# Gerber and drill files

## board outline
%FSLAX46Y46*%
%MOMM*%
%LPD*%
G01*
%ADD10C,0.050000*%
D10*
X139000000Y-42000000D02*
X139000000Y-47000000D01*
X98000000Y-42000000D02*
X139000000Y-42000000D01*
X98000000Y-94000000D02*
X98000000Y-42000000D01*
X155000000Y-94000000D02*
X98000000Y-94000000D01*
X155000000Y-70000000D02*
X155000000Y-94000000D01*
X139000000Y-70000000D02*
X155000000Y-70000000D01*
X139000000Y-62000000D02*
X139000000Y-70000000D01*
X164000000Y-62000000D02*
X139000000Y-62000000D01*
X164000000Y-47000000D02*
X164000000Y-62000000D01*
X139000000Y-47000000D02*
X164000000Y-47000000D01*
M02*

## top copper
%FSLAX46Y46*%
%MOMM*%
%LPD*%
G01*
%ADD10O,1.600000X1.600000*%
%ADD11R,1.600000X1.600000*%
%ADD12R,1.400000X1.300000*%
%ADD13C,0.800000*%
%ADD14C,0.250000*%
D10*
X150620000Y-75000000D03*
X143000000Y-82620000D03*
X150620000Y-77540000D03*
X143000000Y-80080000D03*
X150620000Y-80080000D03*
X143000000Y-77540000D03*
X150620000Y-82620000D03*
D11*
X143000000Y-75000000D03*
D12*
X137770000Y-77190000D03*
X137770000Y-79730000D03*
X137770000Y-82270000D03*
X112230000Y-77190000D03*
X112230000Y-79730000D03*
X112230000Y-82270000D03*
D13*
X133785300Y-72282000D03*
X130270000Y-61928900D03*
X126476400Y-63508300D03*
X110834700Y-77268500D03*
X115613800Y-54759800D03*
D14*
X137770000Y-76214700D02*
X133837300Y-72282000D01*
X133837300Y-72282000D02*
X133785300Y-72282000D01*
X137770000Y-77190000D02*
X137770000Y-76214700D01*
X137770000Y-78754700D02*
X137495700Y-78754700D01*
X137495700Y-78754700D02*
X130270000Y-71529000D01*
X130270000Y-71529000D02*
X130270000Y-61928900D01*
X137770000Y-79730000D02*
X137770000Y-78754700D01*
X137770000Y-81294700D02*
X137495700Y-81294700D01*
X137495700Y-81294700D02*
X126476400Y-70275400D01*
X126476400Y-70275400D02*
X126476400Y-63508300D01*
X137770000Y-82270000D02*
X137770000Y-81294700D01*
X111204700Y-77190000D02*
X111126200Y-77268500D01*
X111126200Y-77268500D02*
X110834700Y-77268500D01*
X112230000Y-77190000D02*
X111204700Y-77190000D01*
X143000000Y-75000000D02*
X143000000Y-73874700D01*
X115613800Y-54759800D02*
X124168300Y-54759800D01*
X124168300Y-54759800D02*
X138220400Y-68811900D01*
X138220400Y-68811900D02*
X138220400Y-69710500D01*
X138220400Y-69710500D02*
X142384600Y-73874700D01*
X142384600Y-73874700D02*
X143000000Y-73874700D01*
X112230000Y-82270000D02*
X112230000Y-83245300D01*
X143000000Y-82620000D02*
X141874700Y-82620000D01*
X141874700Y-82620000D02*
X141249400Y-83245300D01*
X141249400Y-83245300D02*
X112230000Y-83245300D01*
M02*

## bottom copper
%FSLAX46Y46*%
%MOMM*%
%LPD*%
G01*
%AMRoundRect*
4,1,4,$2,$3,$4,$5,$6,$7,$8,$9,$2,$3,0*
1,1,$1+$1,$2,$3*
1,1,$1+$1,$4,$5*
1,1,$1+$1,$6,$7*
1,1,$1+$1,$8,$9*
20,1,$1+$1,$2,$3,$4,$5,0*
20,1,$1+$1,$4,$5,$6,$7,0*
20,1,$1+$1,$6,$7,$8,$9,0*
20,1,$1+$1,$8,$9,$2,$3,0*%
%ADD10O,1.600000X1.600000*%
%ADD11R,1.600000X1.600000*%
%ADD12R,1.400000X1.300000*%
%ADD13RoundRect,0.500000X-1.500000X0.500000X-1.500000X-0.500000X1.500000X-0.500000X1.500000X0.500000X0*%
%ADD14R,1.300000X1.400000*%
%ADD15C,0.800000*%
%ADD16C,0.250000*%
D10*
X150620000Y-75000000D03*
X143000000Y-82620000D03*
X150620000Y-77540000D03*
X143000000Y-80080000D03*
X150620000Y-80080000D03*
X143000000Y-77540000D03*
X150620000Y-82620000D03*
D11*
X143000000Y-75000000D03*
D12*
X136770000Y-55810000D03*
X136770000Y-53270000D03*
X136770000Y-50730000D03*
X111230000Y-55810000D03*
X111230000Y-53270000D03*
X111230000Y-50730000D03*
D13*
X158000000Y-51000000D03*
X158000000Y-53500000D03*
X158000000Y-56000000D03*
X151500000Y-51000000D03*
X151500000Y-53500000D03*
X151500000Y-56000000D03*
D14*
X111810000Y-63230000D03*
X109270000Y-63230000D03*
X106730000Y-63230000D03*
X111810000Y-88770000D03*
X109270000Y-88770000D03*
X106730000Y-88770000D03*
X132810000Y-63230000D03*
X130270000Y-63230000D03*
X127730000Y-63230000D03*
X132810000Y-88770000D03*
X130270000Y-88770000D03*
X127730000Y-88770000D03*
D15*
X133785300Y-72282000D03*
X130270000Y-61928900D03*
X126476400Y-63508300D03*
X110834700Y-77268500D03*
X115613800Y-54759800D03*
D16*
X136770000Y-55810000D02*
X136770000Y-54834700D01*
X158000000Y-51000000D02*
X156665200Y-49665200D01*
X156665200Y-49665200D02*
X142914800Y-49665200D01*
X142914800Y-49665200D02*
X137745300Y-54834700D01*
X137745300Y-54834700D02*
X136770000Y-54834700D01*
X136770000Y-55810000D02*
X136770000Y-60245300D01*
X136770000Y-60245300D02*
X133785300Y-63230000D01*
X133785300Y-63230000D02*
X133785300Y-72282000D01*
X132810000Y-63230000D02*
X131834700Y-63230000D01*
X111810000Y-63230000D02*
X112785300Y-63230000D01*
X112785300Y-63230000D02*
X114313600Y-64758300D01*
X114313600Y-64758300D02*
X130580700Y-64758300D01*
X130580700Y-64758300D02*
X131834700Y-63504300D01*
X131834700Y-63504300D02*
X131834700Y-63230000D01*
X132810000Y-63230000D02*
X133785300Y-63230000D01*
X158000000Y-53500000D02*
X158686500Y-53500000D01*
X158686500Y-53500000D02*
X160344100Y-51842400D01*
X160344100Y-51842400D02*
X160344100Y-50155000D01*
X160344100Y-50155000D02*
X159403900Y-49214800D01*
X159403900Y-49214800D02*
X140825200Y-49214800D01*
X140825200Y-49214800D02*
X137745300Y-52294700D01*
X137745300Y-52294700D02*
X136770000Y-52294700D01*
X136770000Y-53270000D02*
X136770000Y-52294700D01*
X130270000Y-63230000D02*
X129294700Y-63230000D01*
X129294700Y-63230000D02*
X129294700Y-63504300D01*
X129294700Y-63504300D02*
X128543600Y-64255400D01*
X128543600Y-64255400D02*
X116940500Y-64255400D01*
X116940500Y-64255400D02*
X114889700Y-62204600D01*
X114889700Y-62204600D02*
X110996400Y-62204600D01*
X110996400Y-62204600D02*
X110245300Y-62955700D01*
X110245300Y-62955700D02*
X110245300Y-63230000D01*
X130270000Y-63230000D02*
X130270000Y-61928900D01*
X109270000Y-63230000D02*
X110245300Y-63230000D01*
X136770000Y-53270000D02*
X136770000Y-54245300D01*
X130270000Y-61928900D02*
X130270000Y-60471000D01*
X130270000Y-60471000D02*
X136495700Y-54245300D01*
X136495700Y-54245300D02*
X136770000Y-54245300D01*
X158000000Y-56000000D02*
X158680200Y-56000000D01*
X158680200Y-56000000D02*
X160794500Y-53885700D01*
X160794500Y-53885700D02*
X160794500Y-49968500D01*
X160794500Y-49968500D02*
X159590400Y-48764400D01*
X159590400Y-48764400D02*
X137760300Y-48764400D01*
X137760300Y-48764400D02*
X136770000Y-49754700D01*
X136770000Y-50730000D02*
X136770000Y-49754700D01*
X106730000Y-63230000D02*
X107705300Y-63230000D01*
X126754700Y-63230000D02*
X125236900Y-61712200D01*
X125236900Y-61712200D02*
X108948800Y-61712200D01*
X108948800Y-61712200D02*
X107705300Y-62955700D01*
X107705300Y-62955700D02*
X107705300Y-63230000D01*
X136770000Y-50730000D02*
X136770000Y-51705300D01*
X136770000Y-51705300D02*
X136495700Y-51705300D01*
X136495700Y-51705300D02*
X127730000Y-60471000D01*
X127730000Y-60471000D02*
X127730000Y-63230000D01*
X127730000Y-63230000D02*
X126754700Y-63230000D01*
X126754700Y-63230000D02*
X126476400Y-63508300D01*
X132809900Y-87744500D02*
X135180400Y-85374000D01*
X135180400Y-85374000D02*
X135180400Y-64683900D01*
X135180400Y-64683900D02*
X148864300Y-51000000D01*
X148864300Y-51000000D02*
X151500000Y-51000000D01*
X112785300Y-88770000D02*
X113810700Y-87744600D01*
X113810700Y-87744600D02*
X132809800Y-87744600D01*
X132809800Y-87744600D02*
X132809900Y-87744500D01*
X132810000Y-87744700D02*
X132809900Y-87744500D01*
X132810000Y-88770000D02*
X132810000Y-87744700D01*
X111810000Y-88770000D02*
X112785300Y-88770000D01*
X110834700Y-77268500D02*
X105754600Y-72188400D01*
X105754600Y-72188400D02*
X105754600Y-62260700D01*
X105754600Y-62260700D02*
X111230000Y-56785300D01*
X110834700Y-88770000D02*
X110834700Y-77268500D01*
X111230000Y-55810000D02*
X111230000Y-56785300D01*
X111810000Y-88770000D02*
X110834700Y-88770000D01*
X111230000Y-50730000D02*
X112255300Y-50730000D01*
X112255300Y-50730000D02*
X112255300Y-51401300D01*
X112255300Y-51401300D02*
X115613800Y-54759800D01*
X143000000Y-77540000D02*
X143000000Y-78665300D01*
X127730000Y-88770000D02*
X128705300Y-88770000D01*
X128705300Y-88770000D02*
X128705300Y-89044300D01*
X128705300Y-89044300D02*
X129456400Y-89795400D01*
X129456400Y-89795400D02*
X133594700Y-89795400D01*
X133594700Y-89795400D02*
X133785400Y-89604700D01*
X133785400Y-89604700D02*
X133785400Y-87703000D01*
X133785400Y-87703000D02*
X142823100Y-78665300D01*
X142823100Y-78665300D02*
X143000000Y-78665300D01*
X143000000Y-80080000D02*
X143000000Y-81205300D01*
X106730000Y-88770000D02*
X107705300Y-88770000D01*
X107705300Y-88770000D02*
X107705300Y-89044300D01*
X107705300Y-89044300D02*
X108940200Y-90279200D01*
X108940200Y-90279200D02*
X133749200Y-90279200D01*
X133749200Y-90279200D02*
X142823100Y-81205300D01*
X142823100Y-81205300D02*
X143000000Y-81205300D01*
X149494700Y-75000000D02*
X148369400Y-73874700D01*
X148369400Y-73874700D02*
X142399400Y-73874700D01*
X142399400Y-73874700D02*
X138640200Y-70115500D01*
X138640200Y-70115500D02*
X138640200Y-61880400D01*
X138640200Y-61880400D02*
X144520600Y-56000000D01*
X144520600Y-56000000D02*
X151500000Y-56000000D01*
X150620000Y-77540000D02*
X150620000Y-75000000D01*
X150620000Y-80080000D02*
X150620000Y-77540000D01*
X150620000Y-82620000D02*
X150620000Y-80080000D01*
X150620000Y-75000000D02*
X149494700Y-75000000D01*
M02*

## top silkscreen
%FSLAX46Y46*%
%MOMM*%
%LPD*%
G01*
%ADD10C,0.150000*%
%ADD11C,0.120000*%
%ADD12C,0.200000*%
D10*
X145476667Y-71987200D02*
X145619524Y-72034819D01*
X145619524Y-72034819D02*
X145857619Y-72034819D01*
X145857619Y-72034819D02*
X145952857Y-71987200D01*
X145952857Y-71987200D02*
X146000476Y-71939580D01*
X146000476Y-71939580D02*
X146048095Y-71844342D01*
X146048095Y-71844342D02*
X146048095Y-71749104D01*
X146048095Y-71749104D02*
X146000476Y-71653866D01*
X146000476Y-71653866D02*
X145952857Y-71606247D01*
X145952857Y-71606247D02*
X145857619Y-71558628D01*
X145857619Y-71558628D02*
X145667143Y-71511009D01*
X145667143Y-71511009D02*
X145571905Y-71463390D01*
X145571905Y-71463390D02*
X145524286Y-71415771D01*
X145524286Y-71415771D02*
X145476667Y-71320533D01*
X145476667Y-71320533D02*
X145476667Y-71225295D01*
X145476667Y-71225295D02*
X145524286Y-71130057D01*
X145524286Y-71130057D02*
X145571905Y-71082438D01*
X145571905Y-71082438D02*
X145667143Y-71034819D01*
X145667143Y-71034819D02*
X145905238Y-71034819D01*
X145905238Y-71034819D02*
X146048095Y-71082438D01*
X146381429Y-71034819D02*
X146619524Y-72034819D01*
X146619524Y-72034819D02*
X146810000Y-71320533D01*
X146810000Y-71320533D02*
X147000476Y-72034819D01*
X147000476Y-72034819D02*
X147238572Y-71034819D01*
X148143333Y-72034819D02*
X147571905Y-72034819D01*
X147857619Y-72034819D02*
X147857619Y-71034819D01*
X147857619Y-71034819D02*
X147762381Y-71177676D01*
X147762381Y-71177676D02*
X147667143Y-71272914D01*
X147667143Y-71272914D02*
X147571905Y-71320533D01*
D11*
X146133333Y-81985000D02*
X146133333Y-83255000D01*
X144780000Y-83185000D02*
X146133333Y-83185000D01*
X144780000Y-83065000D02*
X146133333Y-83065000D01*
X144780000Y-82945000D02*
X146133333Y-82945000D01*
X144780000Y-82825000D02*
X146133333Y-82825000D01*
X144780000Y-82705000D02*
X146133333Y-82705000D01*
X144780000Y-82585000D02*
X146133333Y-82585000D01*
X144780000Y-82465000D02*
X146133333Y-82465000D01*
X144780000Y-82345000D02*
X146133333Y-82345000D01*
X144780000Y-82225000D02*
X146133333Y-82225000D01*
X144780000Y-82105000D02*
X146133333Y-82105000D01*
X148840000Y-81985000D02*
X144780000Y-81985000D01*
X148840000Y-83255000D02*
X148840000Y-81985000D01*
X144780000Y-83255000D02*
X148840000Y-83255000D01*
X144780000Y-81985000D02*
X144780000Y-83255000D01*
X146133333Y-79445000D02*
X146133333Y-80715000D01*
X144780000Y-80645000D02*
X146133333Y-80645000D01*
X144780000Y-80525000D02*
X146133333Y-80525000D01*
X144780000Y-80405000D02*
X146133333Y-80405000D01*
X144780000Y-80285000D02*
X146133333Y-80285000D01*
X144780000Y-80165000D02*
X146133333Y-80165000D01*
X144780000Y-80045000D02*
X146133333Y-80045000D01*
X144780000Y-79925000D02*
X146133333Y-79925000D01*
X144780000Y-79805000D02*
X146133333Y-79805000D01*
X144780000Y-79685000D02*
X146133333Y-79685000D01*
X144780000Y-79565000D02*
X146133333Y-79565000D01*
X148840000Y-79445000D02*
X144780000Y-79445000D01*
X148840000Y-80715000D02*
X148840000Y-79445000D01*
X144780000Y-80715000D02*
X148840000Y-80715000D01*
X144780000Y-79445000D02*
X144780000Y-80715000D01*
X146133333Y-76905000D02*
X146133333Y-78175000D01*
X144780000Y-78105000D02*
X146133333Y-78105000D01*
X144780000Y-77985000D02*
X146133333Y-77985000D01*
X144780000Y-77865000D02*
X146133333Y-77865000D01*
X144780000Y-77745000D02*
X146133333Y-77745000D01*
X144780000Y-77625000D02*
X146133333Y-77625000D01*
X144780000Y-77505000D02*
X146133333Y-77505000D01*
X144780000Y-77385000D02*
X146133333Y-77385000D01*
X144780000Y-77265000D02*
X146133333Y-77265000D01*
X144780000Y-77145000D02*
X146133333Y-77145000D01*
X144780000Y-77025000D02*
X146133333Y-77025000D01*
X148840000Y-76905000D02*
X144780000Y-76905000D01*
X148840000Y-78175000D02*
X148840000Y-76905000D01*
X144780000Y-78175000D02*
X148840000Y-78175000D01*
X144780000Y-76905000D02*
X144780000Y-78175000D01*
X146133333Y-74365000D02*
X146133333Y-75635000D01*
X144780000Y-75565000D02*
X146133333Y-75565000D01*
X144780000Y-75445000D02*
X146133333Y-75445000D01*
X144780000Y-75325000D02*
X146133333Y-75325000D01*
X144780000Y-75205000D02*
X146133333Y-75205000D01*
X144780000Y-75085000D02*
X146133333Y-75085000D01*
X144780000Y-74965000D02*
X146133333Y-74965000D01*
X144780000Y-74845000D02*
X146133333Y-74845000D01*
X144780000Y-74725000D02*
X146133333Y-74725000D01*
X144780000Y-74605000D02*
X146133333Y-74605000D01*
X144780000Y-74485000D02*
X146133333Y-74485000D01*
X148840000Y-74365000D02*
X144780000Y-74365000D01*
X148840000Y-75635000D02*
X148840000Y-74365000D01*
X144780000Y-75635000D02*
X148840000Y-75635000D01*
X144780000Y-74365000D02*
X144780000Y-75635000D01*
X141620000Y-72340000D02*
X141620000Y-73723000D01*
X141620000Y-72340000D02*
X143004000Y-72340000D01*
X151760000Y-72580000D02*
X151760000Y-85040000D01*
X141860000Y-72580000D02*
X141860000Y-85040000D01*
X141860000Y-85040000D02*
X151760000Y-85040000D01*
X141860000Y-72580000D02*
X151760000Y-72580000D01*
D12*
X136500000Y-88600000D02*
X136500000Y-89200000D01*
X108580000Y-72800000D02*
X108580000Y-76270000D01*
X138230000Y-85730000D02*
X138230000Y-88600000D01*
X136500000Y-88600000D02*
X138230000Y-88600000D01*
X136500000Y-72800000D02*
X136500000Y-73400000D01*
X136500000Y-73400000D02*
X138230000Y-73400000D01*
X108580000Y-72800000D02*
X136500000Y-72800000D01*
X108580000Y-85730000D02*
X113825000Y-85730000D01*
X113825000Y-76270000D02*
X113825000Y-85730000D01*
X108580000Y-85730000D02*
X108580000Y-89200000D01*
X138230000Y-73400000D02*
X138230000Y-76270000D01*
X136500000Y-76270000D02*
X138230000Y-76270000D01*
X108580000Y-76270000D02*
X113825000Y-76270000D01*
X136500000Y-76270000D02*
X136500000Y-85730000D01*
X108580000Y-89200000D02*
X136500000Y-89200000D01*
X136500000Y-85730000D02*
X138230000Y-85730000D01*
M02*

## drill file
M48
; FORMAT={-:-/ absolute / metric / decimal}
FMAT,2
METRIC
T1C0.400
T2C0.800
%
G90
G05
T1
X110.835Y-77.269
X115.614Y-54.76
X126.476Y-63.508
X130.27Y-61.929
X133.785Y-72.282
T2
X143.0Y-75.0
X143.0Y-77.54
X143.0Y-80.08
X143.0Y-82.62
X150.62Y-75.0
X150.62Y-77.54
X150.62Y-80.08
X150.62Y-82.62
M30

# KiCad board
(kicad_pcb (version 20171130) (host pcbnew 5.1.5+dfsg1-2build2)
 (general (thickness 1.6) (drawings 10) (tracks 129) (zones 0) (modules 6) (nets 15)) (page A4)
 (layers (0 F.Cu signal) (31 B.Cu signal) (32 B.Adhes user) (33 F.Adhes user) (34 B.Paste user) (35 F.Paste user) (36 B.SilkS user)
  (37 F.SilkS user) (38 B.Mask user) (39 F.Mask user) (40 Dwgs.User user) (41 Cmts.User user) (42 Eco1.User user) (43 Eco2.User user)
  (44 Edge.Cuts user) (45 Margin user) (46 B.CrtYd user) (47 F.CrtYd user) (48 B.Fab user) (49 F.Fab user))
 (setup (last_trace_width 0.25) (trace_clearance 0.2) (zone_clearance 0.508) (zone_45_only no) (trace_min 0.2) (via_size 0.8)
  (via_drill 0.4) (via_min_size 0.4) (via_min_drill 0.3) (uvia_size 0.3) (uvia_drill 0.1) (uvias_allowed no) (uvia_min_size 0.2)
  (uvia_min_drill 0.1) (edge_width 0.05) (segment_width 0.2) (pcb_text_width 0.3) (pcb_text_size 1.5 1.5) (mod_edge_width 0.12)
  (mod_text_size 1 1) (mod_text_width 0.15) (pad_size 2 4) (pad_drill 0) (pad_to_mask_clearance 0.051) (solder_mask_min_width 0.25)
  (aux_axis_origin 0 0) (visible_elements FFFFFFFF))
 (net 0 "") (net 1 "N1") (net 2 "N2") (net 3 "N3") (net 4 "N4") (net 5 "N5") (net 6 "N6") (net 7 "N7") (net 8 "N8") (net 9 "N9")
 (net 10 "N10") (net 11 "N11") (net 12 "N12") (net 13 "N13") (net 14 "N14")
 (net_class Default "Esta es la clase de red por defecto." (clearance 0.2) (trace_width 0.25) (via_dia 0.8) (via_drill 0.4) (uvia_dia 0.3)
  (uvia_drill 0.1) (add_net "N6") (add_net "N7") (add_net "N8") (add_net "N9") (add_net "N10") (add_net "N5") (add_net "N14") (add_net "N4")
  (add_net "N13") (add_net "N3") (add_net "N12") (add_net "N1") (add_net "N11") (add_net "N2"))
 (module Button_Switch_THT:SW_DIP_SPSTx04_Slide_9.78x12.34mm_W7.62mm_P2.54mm (layer F.Cu) (at 143 75)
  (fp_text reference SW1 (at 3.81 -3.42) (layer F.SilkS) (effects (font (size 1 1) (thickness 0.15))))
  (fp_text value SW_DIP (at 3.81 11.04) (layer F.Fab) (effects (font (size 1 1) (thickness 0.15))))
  (fp_line (start 3.133333 6.985) (end 3.133333 8.255) (layer F.SilkS) (width 0.12))
  (fp_line (start 1.78 8.185) (end 3.133333 8.185) (layer F.SilkS) (width 0.12))
  (fp_line (start 1.78 8.065) (end 3.133333 8.065) (layer F.SilkS) (width 0.12))
  (fp_line (start 1.78 7.945) (end 3.133333 7.945) (layer F.SilkS) (width 0.12))
  (fp_line (start 1.78 7.825) (end 3.133333 7.825) (layer F.SilkS) (width 0.12))
  (fp_line (start 1.78 7.705) (end 3.133333 7.705) (layer F.SilkS) (width 0.12))
  (fp_line (start 1.78 7.585) (end 3.133333 7.585) (layer F.SilkS) (width 0.12))
  (fp_line (start 1.78 7.465) (end 3.133333 7.465) (layer F.SilkS) (width 0.12))
  (fp_line (start 1.78 7.345) (end 3.133333 7.345) (layer F.SilkS) (width 0.12))
  (fp_line (start 1.78 7.225) (end 3.133333 7.225) (layer F.SilkS) (width 0.12))
  (fp_line (start 1.78 7.105) (end 3.133333 7.105) (layer F.SilkS) (width 0.12))
  (fp_line (start 5.84 6.985) (end 1.78 6.985) (layer F.SilkS) (width 0.12))
  (fp_line (start 5.84 8.255) (end 5.84 6.985) (layer F.SilkS) (width 0.12))
  (fp_line (start 1.78 8.255) (end 5.84 8.255) (layer F.SilkS) (width 0.12))
  (fp_line (start 1.78 6.985) (end 1.78 8.255) (layer F.SilkS) (width 0.12))
  (fp_line (start 3.133333 4.445) (end 3.133333 5.715) (layer F.SilkS) (width 0.12))
  (fp_line (start 1.78 5.645) (end 3.133333 5.645) (layer F.SilkS) (width 0.12))
  (fp_line (start 1.78 5.525) (end 3.133333 5.525) (layer F.SilkS) (width 0.12))
  (fp_line (start 1.78 5.405) (end 3.133333 5.405) (layer F.SilkS) (width 0.12))
  (fp_line (start 1.78 5.285) (end 3.133333 5.285) (layer F.SilkS) (width 0.12))
  (fp_line (start 1.78 5.165) (end 3.133333 5.165) (layer F.SilkS) (width 0.12))
  (fp_line (start 1.78 5.045) (end 3.133333 5.045) (layer F.SilkS) (width 0.12))
  (fp_line (start 1.78 4.925) (end 3.133333 4.925) (layer F.SilkS) (width 0.12))
  (fp_line (start 1.78 4.805) (end 3.133333 4.805) (layer F.SilkS) (width 0.12))
  (fp_line (start 1.78 4.685) (end 3.133333 4.685) (layer F.SilkS) (width 0.12))
  (fp_line (start 1.78 4.565) (end 3.133333 4.565) (layer F.SilkS) (width 0.12))
  (fp_line (start 5.84 4.445) (end 1.78 4.445) (layer F.SilkS) (width 0.12))
  (fp_line (start 5.84 5.715) (end 5.84 4.445) (layer F.SilkS) (width 0.12))
  (fp_line (start 1.78 5.715) (end 5.84 5.715) (layer F.SilkS) (width 0.12))
  (fp_line (start 1.78 4.445) (end 1.78 5.715) (layer F.SilkS) (width 0.12))
  (fp_line (start 3.133333 1.905) (end 3.133333 3.175) (layer F.SilkS) (width 0.12))
  (fp_line (start 1.78 3.105) (end 3.133333 3.105) (layer F.SilkS) (width 0.12))
  (fp_line (start 1.78 2.985) (end 3.133333 2.985) (layer F.SilkS) (width 0.12))
  (fp_line (start 1.78 2.865) (end 3.133333 2.865) (layer F.SilkS) (width 0.12))
  (fp_line (start 1.78 2.745) (end 3.133333 2.745) (layer F.SilkS) (width 0.12))
  (fp_line (start 1.78 2.625) (end 3.133333 2.625) (layer F.SilkS) (width 0.12))
  (fp_line (start 1.78 2.505) (end 3.133333 2.505) (layer F.SilkS) (width 0.12))
  (fp_line (start 1.78 2.385) (end 3.133333 2.385) (layer F.SilkS) (width 0.12))
  (fp_line (start 1.78 2.265) (end 3.133333 2.265) (layer F.SilkS) (width 0.12))
  (fp_line (start 1.78 2.145) (end 3.133333 2.145) (layer F.SilkS) (width 0.12))
  (fp_line (start 1.78 2.025) (end 3.133333 2.025) (layer F.SilkS) (width 0.12))
  (fp_line (start 5.84 1.905) (end 1.78 1.905) (layer F.SilkS) (width 0.12))
  (fp_line (start 5.84 3.175) (end 5.84 1.905) (layer F.SilkS) (width 0.12))
  (fp_line (start 1.78 3.175) (end 5.84 3.175) (layer F.SilkS) (width 0.12))
  (fp_line (start 1.78 1.905) (end 1.78 3.175) (layer F.SilkS) (width 0.12))
  (fp_line (start 3.133333 -0.635) (end 3.133333 0.635) (layer F.SilkS) (width 0.12))
  (fp_line (start 1.78 0.565) (end 3.133333 0.565) (layer F.SilkS) (width 0.12))
  (fp_line (start 1.78 0.445) (end 3.133333 0.445) (layer F.SilkS) (width 0.12))
  (fp_line (start 1.78 0.325) (end 3.133333 0.325) (layer F.SilkS) (width 0.12))
  (fp_line (start 1.78 0.205) (end 3.133333 0.205) (layer F.SilkS) (width 0.12))
  (fp_line (start 1.78 0.085) (end 3.133333 0.085) (layer F.SilkS) (width 0.12))
  (fp_line (start 1.78 -0.035) (end 3.133333 -0.035) (layer F.SilkS) (width 0.12))
  (fp_line (start 1.78 -0.155) (end 3.133333 -0.155) (layer F.SilkS) (width 0.12))
  (fp_line (start 1.78 -0.275) (end 3.133333 -0.275) (layer F.SilkS) (width 0.12))
  (fp_line (start 1.78 -0.395) (end 3.133333 -0.395) (layer F.SilkS) (width 0.12))
  (fp_line (start 1.78 -0.515) (end 3.133333 -0.515) (layer F.SilkS) (width 0.12))
  (fp_line (start 5.84 -0.635) (end 1.78 -0.635) (layer F.SilkS) (width 0.12))
  (fp_line (start 5.84 0.635) (end 5.84 -0.635) (layer F.SilkS) (width 0.12))
  (fp_line (start 1.78 0.635) (end 5.84 0.635) (layer F.SilkS) (width 0.12))
  (fp_line (start 1.78 -0.635) (end 1.78 0.635) (layer F.SilkS) (width 0.12))
  (fp_line (start -1.38 -2.66) (end -1.38 -1.277) (layer F.SilkS) (width 0.12))
  (fp_line (start -1.38 -2.66) (end 0.004 -2.66) (layer F.SilkS) (width 0.12))
  (fp_line (start 8.76 -2.42) (end 8.76 10.04) (layer F.SilkS) (width 0.12))
  (fp_line (start -1.14 -2.42) (end -1.14 10.04) (layer F.SilkS) (width 0.12))
  (fp_line (start -1.14 10.04) (end 8.76 10.04) (layer F.SilkS) (width 0.12))
  (fp_line (start -1.14 -2.42) (end 8.76 -2.42) (layer F.SilkS) (width 0.12))
  (pad 8 thru_hole oval (at 7.62 0) (size 1.6 1.6) (drill 0.8) (layers *.Cu *.Mask) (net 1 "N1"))
  (pad 4 thru_hole oval (at 0 7.62) (size 1.6 1.6) (drill 0.8) (layers *.Cu *.Mask) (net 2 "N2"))
  (pad 7 thru_hole oval (at 7.62 2.54) (size 1.6 1.6) (drill 0.8) (layers *.Cu *.Mask) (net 1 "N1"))
  (pad 3 thru_hole oval (at 0 5.08) (size 1.6 1.6) (drill 0.8) (layers *.Cu *.Mask) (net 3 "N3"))
  (pad 6 thru_hole oval (at 7.62 5.08) (size 1.6 1.6) (drill 0.8) (layers *.Cu *.Mask) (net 1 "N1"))
  (pad 2 thru_hole oval (at 0 2.54) (size 1.6 1.6) (drill 0.8) (layers *.Cu *.Mask) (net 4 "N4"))
  (pad 5 thru_hole oval (at 7.62 7.62) (size 1.6 1.6) (drill 0.8) (layers *.Cu *.Mask) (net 1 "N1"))
  (pad 1 thru_hole rect (at 0 0) (size 1.6 1.6) (drill 0.8) (layers *.Cu *.Mask) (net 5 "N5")))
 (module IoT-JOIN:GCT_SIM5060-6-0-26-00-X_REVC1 (layer B.Cu) (at 124 52 90)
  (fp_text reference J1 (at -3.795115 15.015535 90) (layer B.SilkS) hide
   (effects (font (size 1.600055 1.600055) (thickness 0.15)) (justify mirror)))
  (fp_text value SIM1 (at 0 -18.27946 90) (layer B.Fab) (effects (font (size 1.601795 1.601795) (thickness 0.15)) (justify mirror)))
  (pad C1 smd rect (at -3.81 12.77 90) (size 1.3 1.4) (layers B.Cu B.Paste B.Mask) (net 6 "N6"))
  (pad C2 smd rect (at -1.27 12.77 90) (size 1.3 1.4) (layers B.Cu B.Paste B.Mask) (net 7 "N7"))
  (pad C3 smd rect (at 1.27 12.77 90) (size 1.3 1.4) (layers B.Cu B.Paste B.Mask) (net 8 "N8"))
  (pad C5 smd rect (at -3.81 -12.77 90) (size 1.3 1.4) (layers B.Cu B.Paste B.Mask) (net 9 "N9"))
  (pad C6 smd rect (at -1.27 -12.77 90) (size 1.3 1.4) (layers B.Cu B.Paste B.Mask) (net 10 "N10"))
  (pad C7 smd rect (at 1.27 -12.77 90) (size 1.3 1.4) (layers B.Cu B.Paste B.Mask) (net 5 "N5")))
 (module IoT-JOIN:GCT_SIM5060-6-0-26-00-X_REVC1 (layer F.Cu) (at 125 81 270)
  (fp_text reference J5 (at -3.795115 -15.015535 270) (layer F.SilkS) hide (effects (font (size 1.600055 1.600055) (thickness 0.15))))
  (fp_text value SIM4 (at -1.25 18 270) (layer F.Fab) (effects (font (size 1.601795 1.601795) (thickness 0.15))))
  (fp_line (start 7.6 -11.5) (end 8.2 -11.5) (layer F.SilkS) (width 0.2))
  (fp_line (start -8.2 16.42) (end -4.73 16.42) (layer F.SilkS) (width 0.2))
  (fp_line (start 4.73 -13.23) (end 7.6 -13.23) (layer F.SilkS) (width 0.2))
  (fp_line (start 7.6 -11.5) (end 7.6 -13.23) (layer F.SilkS) (width 0.2))
  (fp_line (start -8.2 -11.5) (end -7.6 -11.5) (layer F.SilkS) (width 0.2))
  (fp_line (start -7.6 -11.5) (end -7.6 -13.23) (layer F.SilkS) (width 0.2))
  (fp_line (start -8.2 16.42) (end -8.2 -11.5) (layer F.SilkS) (width 0.2))
  (fp_line (start 4.73 16.42) (end 4.73 11.175) (layer F.SilkS) (width 0.2))
  (fp_line (start -4.73 11.175) (end 4.73 11.175) (layer F.SilkS) (width 0.2))
  (fp_line (start 4.73 16.42) (end 8.2 16.42) (layer F.SilkS) (width 0.2))
  (fp_line (start -7.6 -13.23) (end -4.73 -13.23) (layer F.SilkS) (width 0.2))
  (fp_line (start -4.73 -11.5) (end -4.73 -13.23) (layer F.SilkS) (width 0.2))
  (fp_line (start -4.73 16.42) (end -4.73 11.175) (layer F.SilkS) (width 0.2))
  (fp_line (start -4.73 -11.5) (end 4.73 -11.5) (layer F.SilkS) (width 0.2))
  (fp_line (start 8.2 16.42) (end 8.2 -11.5) (layer F.SilkS) (width 0.2))
  (fp_line (start 4.73 -11.5) (end 4.73 -13.23) (layer F.SilkS) (width 0.2))
  (pad C1 smd rect (at -3.81 -12.77 270) (size 1.3 1.4) (layers F.Cu F.Paste F.Mask) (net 6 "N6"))
  (pad C2 smd rect (at -1.27 -12.77 270) (size 1.3 1.4) (layers F.Cu F.Paste F.Mask) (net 7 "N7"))
  (pad C3 smd rect (at 1.27 -12.77 270) (size 1.3 1.4) (layers F.Cu F.Paste F.Mask) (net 8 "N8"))
  (pad C5 smd rect (at -3.81 12.77 270) (size 1.3 1.4) (layers F.Cu F.Paste F.Mask) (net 9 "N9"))
  (pad C6 smd rect (at -1.27 12.77 270) (size 1.3 1.4) (layers F.Cu F.Paste F.Mask) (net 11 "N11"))
  (pad C7 smd rect (at 1.27 12.77 270) (size 1.3 1.4) (layers F.Cu F.Paste F.Mask) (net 2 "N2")))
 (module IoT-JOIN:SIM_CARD (layer B.Cu) (at 164 47 270)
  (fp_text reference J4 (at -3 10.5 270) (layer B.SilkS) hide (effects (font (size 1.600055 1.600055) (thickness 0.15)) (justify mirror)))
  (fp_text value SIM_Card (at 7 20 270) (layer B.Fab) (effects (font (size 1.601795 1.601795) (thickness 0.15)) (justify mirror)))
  (pad 1 connect roundrect (at 4 6 270) (size 2 4) (layers B.Cu B.Mask) (roundrect_rratio 0.25) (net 6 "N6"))
  (pad 2 connect roundrect (at 6.5 6 270) (size 2 4) (layers B.Cu B.Mask) (roundrect_rratio 0.25) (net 7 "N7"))
  (pad 3 connect roundrect (at 9 6 270) (size 2 4) (layers B.Cu B.Mask) (roundrect_rratio 0.25) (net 8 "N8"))
  (pad 5 connect roundrect (at 4 12.5 270) (size 2 4) (layers B.Cu B.Mask) (roundrect_rratio 0.25) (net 9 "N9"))
  (pad 6 connect roundrect (at 6.5 12.5 270) (size 2 4) (layers B.Cu B.Mask) (roundrect_rratio 0.25) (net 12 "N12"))
  (pad 7 connect roundrect (at 9 12.5 270) (size 2 4) (layers B.Cu B.Mask) (roundrect_rratio 0.25) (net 1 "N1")))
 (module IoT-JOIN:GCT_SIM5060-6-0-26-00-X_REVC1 (layer B.Cu) (at 108 76 180)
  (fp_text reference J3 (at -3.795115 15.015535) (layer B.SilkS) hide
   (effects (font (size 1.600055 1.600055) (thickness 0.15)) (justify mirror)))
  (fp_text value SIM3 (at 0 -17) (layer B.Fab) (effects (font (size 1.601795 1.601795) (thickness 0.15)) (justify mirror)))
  (pad C1 smd rect (at -3.81 12.77 180) (size 1.3 1.4) (layers B.Cu B.Paste B.Mask) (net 6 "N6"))
  (pad C2 smd rect (at -1.27 12.77 180) (size 1.3 1.4) (layers B.Cu B.Paste B.Mask) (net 7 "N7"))
  (pad C3 smd rect (at 1.27 12.77 180) (size 1.3 1.4) (layers B.Cu B.Paste B.Mask) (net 8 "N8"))
  (pad C5 smd rect (at -3.81 -12.77 180) (size 1.3 1.4) (layers B.Cu B.Paste B.Mask) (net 9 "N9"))
  (pad C6 smd rect (at -1.27 -12.77 180) (size 1.3 1.4) (layers B.Cu B.Paste B.Mask) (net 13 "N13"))
  (pad C7 smd rect (at 1.27 -12.77 180) (size 1.3 1.4) (layers B.Cu B.Paste B.Mask) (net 3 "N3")))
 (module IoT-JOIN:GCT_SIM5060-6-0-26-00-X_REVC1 (layer B.Cu) (at 129 76 180)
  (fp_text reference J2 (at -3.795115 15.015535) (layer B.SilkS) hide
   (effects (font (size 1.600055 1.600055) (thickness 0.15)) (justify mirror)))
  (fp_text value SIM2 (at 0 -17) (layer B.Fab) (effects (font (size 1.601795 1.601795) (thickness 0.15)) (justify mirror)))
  (pad C1 smd rect (at -3.81 12.77 180) (size 1.3 1.4) (layers B.Cu B.Paste B.Mask) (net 6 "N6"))
  (pad C2 smd rect (at -1.27 12.77 180) (size 1.3 1.4) (layers B.Cu B.Paste B.Mask) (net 7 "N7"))
  (pad C3 smd rect (at 1.27 12.77 180) (size 1.3 1.4) (layers B.Cu B.Paste B.Mask) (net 8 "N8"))
  (pad C5 smd rect (at -3.81 -12.77 180) (size 1.3 1.4) (layers B.Cu B.Paste B.Mask) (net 9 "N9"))
  (pad C6 smd rect (at -1.27 -12.77 180) (size 1.3 1.4) (layers B.Cu B.Paste B.Mask) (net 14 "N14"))
  (pad C7 smd rect (at 1.27 -12.77 180) (size 1.3 1.4) (layers B.Cu B.Paste B.Mask) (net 4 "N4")))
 (gr_line (start 139 42) (end 139 47) (layer Edge.Cuts) (width 0.05))
 (gr_line (start 98 42) (end 139 42) (layer Edge.Cuts) (width 0.05))
 (gr_line (start 98 94) (end 98 42) (layer Edge.Cuts) (width 0.05))
 (gr_line (start 155 94) (end 98 94) (layer Edge.Cuts) (width 0.05))
 (gr_line (start 155 70) (end 155 94) (layer Edge.Cuts) (width 0.05))
 (gr_line (start 139 70) (end 155 70) (layer Edge.Cuts) (width 0.05))
 (gr_line (start 139 62) (end 139 70) (layer Edge.Cuts) (width 0.05))
 (gr_line (start 164 62) (end 139 62) (layer Edge.Cuts) (width 0.05))
 (gr_line (start 164 47) (end 164 62) (layer Edge.Cuts) (width 0.05))
 (gr_line (start 139 47) (end 164 47) (layer Edge.Cuts) (width 0.05))
 (segment (start 136.77 55.81) (end 136.77 54.8347) (width 0.25) (layer B.Cu) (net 6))
 (segment (start 158 51) (end 156.6652 49.6652) (width 0.25) (layer B.Cu) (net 6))
 (segment (start 156.6652 49.6652) (end 142.9148 49.6652) (width 0.25) (layer B.Cu) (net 6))
 (segment (start 142.9148 49.6652) (end 137.7453 54.8347) (width 0.25) (layer B.Cu) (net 6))
 (segment (start 137.7453 54.8347) (end 136.77 54.8347) (width 0.25) (layer B.Cu) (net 6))
 (segment (start 136.77 55.81) (end 136.77 60.2453) (width 0.25) (layer B.Cu) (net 6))
 (segment (start 136.77 60.2453) (end 133.7853 63.23) (width 0.25) (layer B.Cu) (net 6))
 (segment (start 137.77 76.2147) (end 133.8373 72.282) (width 0.25) (layer F.Cu) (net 6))
 (segment (start 133.8373 72.282) (end 133.7853 72.282) (width 0.25) (layer F.Cu) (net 6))
 (segment (start 133.7853 63.23) (end 133.7853 72.282) (width 0.25) (layer B.Cu) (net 6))
 (segment (start 137.77 77.19) (end 137.77 76.2147) (width 0.25) (layer F.Cu) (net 6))
 (segment (start 132.81 63.23) (end 131.8347 63.23) (width 0.25) (layer B.Cu) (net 6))
 (segment (start 111.81 63.23) (end 112.7853 63.23) (width 0.25) (layer B.Cu) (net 6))
 (segment (start 112.7853 63.23) (end 114.3136 64.7583) (width 0.25) (layer B.Cu) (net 6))
 (segment (start 114.3136 64.7583) (end 130.5807 64.7583) (width 0.25) (layer B.Cu) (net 6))
 (segment (start 130.5807 64.7583) (end 131.8347 63.5043) (width 0.25) (layer B.Cu) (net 6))
 (segment (start 131.8347 63.5043) (end 131.8347 63.23) (width 0.25) (layer B.Cu) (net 6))
 (segment (start 132.81 63.23) (end 133.7853 63.23) (width 0.25) (layer B.Cu) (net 6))
 (via (at 133.7853 72.282) (size 0.8) (layers F.Cu B.Cu) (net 6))
 (segment (start 158 53.5) (end 158.6865 53.5) (width 0.25) (layer B.Cu) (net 7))
 (segment (start 158.6865 53.5) (end 160.3441 51.8424) (width 0.25) (layer B.Cu) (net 7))
 (segment (start 160.3441 51.8424) (end 160.3441 50.155) (width 0.25) (layer B.Cu) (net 7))
 (segment (start 160.3441 50.155) (end 159.4039 49.2148) (width 0.25) (layer B.Cu) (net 7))
 (segment (start 159.4039 49.2148) (end 140.8252 49.2148) (width 0.25) (layer B.Cu) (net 7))
 (segment (start 140.8252 49.2148) (end 137.7453 52.2947) (width 0.25) (layer B.Cu) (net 7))
 (segment (start 137.7453 52.2947) (end 136.77 52.2947) (width 0.25) (layer B.Cu) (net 7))
 (segment (start 136.77 53.27) (end 136.77 52.2947) (width 0.25) (layer B.Cu) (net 7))
 (segment (start 130.27 63.23) (end 129.2947 63.23) (width 0.25) (layer B.Cu) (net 7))
 (segment (start 129.2947 63.23) (end 129.2947 63.5043) (width 0.25) (layer B.Cu) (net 7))
 (segment (start 129.2947 63.5043) (end 128.5436 64.2554) (width 0.25) (layer B.Cu) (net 7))
 (segment (start 128.5436 64.2554) (end 116.9405 64.2554) (width 0.25) (layer B.Cu) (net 7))
 (segment (start 116.9405 64.2554) (end 114.8897 62.2046) (width 0.25) (layer B.Cu) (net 7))
 (segment (start 114.8897 62.2046) (end 110.9964 62.2046) (width 0.25) (layer B.Cu) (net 7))
 (segment (start 110.9964 62.2046) (end 110.2453 62.9557) (width 0.25) (layer B.Cu) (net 7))
 (segment (start 110.2453 62.9557) (end 110.2453 63.23) (width 0.25) (layer B.Cu) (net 7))
 (segment (start 130.27 63.23) (end 130.27 61.9289) (width 0.25) (layer B.Cu) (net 7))
 (segment (start 109.27 63.23) (end 110.2453 63.23) (width 0.25) (layer B.Cu) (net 7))
 (segment (start 136.77 53.27) (end 136.77 54.2453) (width 0.25) (layer B.Cu) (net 7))
 (segment (start 130.27 61.9289) (end 130.27 60.471) (width 0.25) (layer B.Cu) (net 7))
 (segment (start 130.27 60.471) (end 136.4957 54.2453) (width 0.25) (layer B.Cu) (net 7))
 (segment (start 136.4957 54.2453) (end 136.77 54.2453) (width 0.25) (layer B.Cu) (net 7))
 (segment (start 137.77 78.7547) (end 137.4957 78.7547) (width 0.25) (layer F.Cu) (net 7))
 (segment (start 137.4957 78.7547) (end 130.27 71.529) (width 0.25) (layer F.Cu) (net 7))
 (segment (start 130.27 71.529) (end 130.27 61.9289) (width 0.25) (layer F.Cu) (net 7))
 (segment (start 137.77 79.73) (end 137.77 78.7547) (width 0.25) (layer F.Cu) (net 7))
 (via (at 130.27 61.9289) (size 0.8) (layers F.Cu B.Cu) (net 7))
 (segment (start 158 56) (end 158.6802 56) (width 0.25) (layer B.Cu) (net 8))
 (segment (start 158.6802 56) (end 160.7945 53.8857) (width 0.25) (layer B.Cu) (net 8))
 (segment (start 160.7945 53.8857) (end 160.7945 49.9685) (width 0.25) (layer B.Cu) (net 8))
 (segment (start 160.7945 49.9685) (end 159.5904 48.7644) (width 0.25) (layer B.Cu) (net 8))
 (segment (start 159.5904 48.7644) (end 137.7603 48.7644) (width 0.25) (layer B.Cu) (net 8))
 (segment (start 137.7603 48.7644) (end 136.77 49.7547) (width 0.25) (layer B.Cu) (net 8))
 (segment (start 136.77 50.73) (end 136.77 49.7547) (width 0.25) (layer B.Cu) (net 8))
 (segment (start 106.73 63.23) (end 107.7053 63.23) (width 0.25) (layer B.Cu) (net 8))
 (segment (start 126.7547 63.23) (end 125.2369 61.7122) (width 0.25) (layer B.Cu) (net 8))
 (segment (start 125.2369 61.7122) (end 108.9488 61.7122) (width 0.25) (layer B.Cu) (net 8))
 (segment (start 108.9488 61.7122) (end 107.7053 62.9557) (width 0.25) (layer B.Cu) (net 8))
 (segment (start 107.7053 62.9557) (end 107.7053 63.23) (width 0.25) (layer B.Cu) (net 8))
 (segment (start 136.77 50.73) (end 136.77 51.7053) (width 0.25) (layer B.Cu) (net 8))
 (segment (start 136.77 51.7053) (end 136.4957 51.7053) (width 0.25) (layer B.Cu) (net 8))
 (segment (start 136.4957 51.7053) (end 127.73 60.471) (width 0.25) (layer B.Cu) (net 8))
 (segment (start 127.73 60.471) (end 127.73 63.23) (width 0.25) (layer B.Cu) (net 8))
 (segment (start 127.73 63.23) (end 126.7547 63.23) (width 0.25) (layer B.Cu) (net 8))
 (segment (start 137.77 81.2947) (end 137.4957 81.2947) (width 0.25) (layer F.Cu) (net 8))
 (segment (start 137.4957 81.2947) (end 126.4764 70.2754) (width 0.25) (layer F.Cu) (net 8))
 (segment (start 126.4764 70.2754) (end 126.4764 63.5083) (width 0.25) (layer F.Cu) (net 8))
 (segment (start 126.7547 63.23) (end 126.4764 63.5083) (width 0.25) (layer B.Cu) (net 8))
 (segment (start 137.77 82.27) (end 137.77 81.2947) (width 0.25) (layer F.Cu) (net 8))
 (via (at 126.4764 63.5083) (size 0.8) (layers F.Cu B.Cu) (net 8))
 (segment (start 132.8099 87.7445) (end 135.1804 85.374) (width 0.25) (layer B.Cu) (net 9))
 (segment (start 135.1804 85.374) (end 135.1804 64.6839) (width 0.25) (layer B.Cu) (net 9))
 (segment (start 135.1804 64.6839) (end 148.8643 51) (width 0.25) (layer B.Cu) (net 9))
 (segment (start 148.8643 51) (end 151.5 51) (width 0.25) (layer B.Cu) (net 9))
 (segment (start 112.7853 88.77) (end 113.8107 87.7446) (width 0.25) (layer B.Cu) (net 9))
 (segment (start 113.8107 87.7446) (end 132.8098 87.7446) (width 0.25) (layer B.Cu) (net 9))
 (segment (start 132.8098 87.7446) (end 132.8099 87.7445) (width 0.25) (layer B.Cu) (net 9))
 (segment (start 132.81 87.7447) (end 132.8099 87.7445) (width 0.25) (layer B.Cu) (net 9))
 (segment (start 132.81 88.77) (end 132.81 87.7447) (width 0.25) (layer B.Cu) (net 9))
 (segment (start 111.81 88.77) (end 112.7853 88.77) (width 0.25) (layer B.Cu) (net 9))
 (segment (start 110.8347 77.2685) (end 105.7546 72.1884) (width 0.25) (layer B.Cu) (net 9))
 (segment (start 105.7546 72.1884) (end 105.7546 62.2607) (width 0.25) (layer B.Cu) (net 9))
 (segment (start 105.7546 62.2607) (end 111.23 56.7853) (width 0.25) (layer B.Cu) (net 9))
 (segment (start 110.8347 88.77) (end 110.8347 77.2685) (width 0.25) (layer B.Cu) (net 9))
 (segment (start 111.23 55.81) (end 111.23 56.7853) (width 0.25) (layer B.Cu) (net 9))
 (segment (start 111.2047 77.19) (end 111.1262 77.2685) (width 0.25) (layer F.Cu) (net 9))
 (segment (start 111.1262 77.2685) (end 110.8347 77.2685) (width 0.25) (layer F.Cu) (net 9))
 (segment (start 111.81 88.77) (end 110.8347 88.77) (width 0.25) (layer B.Cu) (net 9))
 (segment (start 112.23 77.19) (end 111.2047 77.19) (width 0.25) (layer F.Cu) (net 9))
 (via (at 110.8347 77.2685) (size 0.8) (layers F.Cu B.Cu) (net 9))
 (segment (start 111.23 50.73) (end 112.2553 50.73) (width 0.25) (layer B.Cu) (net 5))
 (segment (start 143 75) (end 143 73.8747) (width 0.25) (layer F.Cu) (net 5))
 (segment (start 115.6138 54.7598) (end 124.1683 54.7598) (width 0.25) (layer F.Cu) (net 5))
 (segment (start 124.1683 54.7598) (end 138.2204 68.8119) (width 0.25) (layer F.Cu) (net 5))
 (segment (start 138.2204 68.8119) (end 138.2204 69.7105) (width 0.25) (layer F.Cu) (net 5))
 (segment (start 138.2204 69.7105) (end 142.3846 73.8747) (width 0.25) (layer F.Cu) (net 5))
 (segment (start 142.3846 73.8747) (end 143 73.8747) (width 0.25) (layer F.Cu) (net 5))
 (segment (start 112.2553 50.73) (end 112.2553 51.4013) (width 0.25) (layer B.Cu) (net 5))
 (segment (start 112.2553 51.4013) (end 115.6138 54.7598) (width 0.25) (layer B.Cu) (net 5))
 (via (at 115.6138 54.7598) (size 0.8) (layers F.Cu B.Cu) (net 5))
 (segment (start 143 77.54) (end 143 78.6653) (width 0.25) (layer B.Cu) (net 4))
 (segment (start 127.73 88.77) (end 128.7053 88.77) (width 0.25) (layer B.Cu) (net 4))
 (segment (start 128.7053 88.77) (end 128.7053 89.0443) (width 0.25) (layer B.Cu) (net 4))
 (segment (start 128.7053 89.0443) (end 129.4564 89.7954) (width 0.25) (layer B.Cu) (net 4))
 (segment (start 129.4564 89.7954) (end 133.5947 89.7954) (width 0.25) (layer B.Cu) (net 4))
 (segment (start 133.5947 89.7954) (end 133.7854 89.6047) (width 0.25) (layer B.Cu) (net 4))
 (segment (start 133.7854 89.6047) (end 133.7854 87.703) (width 0.25) (layer B.Cu) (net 4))
 (segment (start 133.7854 87.703) (end 142.8231 78.6653) (width 0.25) (layer B.Cu) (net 4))
 (segment (start 142.8231 78.6653) (end 143 78.6653) (width 0.25) (layer B.Cu) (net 4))
 (segment (start 143 80.08) (end 143 81.2053) (width 0.25) (layer B.Cu) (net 3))
 (segment (start 106.73 88.77) (end 107.7053 88.77) (width 0.25) (layer B.Cu) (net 3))
 (segment (start 107.7053 88.77) (end 107.7053 89.0443) (width 0.25) (layer B.Cu) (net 3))
 (segment (start 107.7053 89.0443) (end 108.9402 90.2792) (width 0.25) (layer B.Cu) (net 3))
 (segment (start 108.9402 90.2792) (end 133.7492 90.2792) (width 0.25) (layer B.Cu) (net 3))
 (segment (start 133.7492 90.2792) (end 142.8231 81.2053) (width 0.25) (layer B.Cu) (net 3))
 (segment (start 142.8231 81.2053) (end 143 81.2053) (width 0.25) (layer B.Cu) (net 3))
 (segment (start 149.4947 75) (end 148.3694 73.8747) (width 0.25) (layer B.Cu) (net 1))
 (segment (start 148.3694 73.8747) (end 142.3994 73.8747) (width 0.25) (layer B.Cu) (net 1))
 (segment (start 142.3994 73.8747) (end 138.6402 70.1155) (width 0.25) (layer B.Cu) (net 1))
 (segment (start 138.6402 70.1155) (end 138.6402 61.8804) (width 0.25) (layer B.Cu) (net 1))
 (segment (start 138.6402 61.8804) (end 144.5206 56) (width 0.25) (layer B.Cu) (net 1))
 (segment (start 144.5206 56) (end 151.5 56) (width 0.25) (layer B.Cu) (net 1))
 (segment (start 150.62 77.54) (end 150.62 75) (width 0.25) (layer B.Cu) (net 1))
 (segment (start 150.62 80.08) (end 150.62 77.54) (width 0.25) (layer B.Cu) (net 1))
 (segment (start 150.62 82.62) (end 150.62 80.08) (width 0.25) (layer B.Cu) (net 1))
 (segment (start 150.62 75) (end 149.4947 75) (width 0.25) (layer B.Cu) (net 1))
 (segment (start 112.23 82.27) (end 112.23 83.2453) (width 0.25) (layer F.Cu) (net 2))
 (segment (start 143 82.62) (end 141.8747 82.62) (width 0.25) (layer F.Cu) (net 2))
 (segment (start 141.8747 82.62) (end 141.2494 83.2453) (width 0.25) (layer F.Cu) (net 2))
 (segment (start 141.2494 83.2453) (end 112.23 83.2453) (width 0.25) (layer F.Cu) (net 2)))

